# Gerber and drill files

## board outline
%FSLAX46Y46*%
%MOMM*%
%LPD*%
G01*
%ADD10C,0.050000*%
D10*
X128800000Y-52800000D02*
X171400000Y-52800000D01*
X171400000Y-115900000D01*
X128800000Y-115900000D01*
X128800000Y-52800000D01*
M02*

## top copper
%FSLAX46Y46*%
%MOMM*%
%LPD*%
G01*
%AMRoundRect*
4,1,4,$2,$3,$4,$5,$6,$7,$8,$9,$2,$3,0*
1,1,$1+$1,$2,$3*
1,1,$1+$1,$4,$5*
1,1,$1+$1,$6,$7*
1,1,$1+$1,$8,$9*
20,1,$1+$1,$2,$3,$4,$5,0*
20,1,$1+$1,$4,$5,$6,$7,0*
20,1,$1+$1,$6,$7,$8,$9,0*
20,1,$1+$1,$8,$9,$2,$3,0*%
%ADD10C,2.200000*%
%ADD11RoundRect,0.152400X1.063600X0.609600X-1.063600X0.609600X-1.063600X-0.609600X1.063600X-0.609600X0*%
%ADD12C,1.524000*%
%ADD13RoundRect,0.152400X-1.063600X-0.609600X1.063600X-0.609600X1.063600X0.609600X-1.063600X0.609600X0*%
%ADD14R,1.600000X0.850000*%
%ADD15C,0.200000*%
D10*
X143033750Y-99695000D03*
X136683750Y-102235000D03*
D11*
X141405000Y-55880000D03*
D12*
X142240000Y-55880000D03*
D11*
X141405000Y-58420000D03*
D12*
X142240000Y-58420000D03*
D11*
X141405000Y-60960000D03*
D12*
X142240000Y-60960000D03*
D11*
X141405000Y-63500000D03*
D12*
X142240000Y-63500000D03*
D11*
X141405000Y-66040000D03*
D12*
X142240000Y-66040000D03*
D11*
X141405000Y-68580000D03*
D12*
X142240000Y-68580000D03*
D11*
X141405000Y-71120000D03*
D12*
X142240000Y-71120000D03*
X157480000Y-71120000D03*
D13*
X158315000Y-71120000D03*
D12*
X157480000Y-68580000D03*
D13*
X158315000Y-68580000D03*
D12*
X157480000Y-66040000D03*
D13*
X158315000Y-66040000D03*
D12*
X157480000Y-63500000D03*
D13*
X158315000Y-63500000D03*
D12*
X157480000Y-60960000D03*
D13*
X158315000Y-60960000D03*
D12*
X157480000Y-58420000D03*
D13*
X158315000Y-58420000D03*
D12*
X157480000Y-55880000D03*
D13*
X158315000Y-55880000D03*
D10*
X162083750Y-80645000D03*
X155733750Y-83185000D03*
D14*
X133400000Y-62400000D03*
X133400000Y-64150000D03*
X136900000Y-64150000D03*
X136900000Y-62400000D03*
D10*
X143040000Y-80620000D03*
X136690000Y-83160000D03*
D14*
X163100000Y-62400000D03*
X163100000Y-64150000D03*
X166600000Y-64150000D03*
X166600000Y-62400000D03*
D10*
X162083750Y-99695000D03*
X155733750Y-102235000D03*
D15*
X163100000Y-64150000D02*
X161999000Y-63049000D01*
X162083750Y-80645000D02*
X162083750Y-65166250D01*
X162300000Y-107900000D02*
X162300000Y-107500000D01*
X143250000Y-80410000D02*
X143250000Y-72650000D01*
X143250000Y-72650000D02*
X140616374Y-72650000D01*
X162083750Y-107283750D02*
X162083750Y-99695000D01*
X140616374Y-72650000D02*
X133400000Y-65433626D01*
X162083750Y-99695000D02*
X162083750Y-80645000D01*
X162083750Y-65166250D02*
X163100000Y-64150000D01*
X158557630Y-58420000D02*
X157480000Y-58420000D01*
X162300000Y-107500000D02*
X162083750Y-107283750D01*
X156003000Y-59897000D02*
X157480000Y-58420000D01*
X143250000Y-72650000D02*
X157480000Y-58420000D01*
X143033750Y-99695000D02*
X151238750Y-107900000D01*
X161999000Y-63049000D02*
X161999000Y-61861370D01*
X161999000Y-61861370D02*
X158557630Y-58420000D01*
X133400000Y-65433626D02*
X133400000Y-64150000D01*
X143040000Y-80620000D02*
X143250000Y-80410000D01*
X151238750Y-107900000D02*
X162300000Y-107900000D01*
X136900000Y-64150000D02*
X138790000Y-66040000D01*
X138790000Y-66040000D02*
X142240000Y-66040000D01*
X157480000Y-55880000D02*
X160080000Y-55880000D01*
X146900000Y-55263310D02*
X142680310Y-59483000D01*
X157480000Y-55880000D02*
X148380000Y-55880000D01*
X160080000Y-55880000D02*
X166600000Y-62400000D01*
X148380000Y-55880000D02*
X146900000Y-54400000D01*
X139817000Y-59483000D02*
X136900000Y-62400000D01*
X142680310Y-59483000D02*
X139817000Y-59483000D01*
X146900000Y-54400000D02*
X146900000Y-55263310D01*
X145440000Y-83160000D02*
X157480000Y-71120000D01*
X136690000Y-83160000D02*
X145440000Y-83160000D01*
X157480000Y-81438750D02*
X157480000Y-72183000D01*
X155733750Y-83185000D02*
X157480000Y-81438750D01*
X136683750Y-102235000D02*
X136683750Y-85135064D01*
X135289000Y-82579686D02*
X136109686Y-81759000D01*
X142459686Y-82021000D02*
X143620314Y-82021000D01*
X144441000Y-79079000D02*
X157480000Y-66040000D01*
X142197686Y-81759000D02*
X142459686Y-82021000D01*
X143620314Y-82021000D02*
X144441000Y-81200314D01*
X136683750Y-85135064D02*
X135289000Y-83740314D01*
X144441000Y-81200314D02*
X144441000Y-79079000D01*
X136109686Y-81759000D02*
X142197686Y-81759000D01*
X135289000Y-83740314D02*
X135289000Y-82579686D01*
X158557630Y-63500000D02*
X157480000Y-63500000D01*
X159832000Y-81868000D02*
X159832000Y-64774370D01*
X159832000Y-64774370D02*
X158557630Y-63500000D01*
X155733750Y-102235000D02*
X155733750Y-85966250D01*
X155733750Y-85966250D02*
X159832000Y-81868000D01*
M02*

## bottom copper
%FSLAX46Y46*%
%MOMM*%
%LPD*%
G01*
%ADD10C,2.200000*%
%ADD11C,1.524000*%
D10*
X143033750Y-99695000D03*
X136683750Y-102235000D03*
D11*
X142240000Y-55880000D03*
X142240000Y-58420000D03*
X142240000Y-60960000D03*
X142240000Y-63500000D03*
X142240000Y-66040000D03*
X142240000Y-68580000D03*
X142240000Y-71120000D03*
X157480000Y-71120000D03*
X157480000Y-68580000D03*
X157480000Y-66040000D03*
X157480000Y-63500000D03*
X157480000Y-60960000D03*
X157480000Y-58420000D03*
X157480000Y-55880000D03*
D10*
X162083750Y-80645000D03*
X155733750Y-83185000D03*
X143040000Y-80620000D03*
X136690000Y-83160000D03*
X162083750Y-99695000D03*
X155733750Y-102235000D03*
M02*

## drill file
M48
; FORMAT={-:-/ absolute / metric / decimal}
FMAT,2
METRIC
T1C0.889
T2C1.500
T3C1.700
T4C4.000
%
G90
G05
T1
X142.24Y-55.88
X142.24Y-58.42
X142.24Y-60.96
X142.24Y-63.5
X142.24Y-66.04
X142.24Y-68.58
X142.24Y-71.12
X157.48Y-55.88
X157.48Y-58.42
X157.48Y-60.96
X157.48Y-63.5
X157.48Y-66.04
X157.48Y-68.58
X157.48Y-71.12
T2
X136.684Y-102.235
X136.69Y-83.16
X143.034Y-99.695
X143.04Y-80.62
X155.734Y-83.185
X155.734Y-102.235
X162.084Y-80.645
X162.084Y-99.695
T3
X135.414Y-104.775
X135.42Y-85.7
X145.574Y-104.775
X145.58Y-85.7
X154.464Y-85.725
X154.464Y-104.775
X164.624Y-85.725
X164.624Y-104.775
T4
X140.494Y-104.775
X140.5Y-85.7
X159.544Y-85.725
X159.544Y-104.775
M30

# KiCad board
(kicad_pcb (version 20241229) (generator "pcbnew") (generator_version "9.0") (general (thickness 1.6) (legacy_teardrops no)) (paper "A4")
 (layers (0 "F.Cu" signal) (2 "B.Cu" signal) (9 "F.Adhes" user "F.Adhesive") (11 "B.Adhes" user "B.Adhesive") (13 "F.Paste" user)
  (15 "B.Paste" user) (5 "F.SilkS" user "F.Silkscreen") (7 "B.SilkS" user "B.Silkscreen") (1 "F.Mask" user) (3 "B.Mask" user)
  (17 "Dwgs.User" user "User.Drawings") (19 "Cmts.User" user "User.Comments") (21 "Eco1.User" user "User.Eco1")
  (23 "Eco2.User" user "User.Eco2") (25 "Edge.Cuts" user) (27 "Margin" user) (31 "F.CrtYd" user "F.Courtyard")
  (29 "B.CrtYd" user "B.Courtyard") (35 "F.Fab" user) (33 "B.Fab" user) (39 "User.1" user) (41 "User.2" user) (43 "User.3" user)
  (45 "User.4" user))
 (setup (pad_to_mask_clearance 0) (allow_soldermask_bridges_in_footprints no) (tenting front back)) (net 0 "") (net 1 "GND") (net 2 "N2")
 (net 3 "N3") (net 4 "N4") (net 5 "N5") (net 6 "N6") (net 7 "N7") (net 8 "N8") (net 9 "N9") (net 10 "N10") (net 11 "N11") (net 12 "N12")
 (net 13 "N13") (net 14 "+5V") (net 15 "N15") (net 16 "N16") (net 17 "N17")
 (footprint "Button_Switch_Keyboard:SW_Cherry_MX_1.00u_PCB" (layer "F.Cu") (at 143.03375 99.695)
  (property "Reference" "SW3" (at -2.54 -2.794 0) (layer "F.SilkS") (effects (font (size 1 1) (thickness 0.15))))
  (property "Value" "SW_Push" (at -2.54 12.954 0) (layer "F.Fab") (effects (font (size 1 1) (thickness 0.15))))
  (pad "" np_thru_hole circle (at -7.62 5.08) (size 1.7 1.7) (drill 1.7) (layers "*.Cu" "*.Mask"))
  (pad "" np_thru_hole circle (at -2.54 5.08) (size 4 4) (drill 4) (layers "*.Cu" "*.Mask"))
  (pad "" np_thru_hole circle (at 2.54 5.08) (size 1.7 1.7) (drill 1.7) (layers "*.Cu" "*.Mask"))
  (pad "1" thru_hole circle (at 0 0) (size 2.2 2.2) (drill 1.5) (layers "*.Cu" "*.Mask") (remove_unused_layers no) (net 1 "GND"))
  (pad "2" thru_hole circle (at -6.35 2.54) (size 2.2 2.2) (drill 1.5) (layers "*.Cu" "*.Mask") (remove_unused_layers no) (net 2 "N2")))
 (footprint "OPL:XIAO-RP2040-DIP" (layer "F.Cu") (at 149.86 63.5)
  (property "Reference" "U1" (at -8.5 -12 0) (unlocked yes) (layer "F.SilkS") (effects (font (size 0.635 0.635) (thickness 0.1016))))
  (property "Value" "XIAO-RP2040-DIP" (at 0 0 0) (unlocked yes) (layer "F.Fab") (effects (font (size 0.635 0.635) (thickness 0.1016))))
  (pad "1" smd roundrect (at -8.455 -7.62 180) (size 2.432 1.524) (layers "F.Cu" "F.Mask") (roundrect_rratio 0.1) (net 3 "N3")
   (thermal_bridge_angle 45))
  (pad "1" thru_hole circle (at -7.62 -7.62 180) (size 1.524 1.524) (drill 0.889) (layers "*.Cu" "*.Mask") (remove_unused_layers no)
   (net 3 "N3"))
  (pad "2" smd roundrect (at -8.455 -5.08 180) (size 2.432 1.524) (layers "F.Cu" "F.Mask") (roundrect_rratio 0.1) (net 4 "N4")
   (thermal_bridge_angle 45))
  (pad "2" thru_hole circle (at -7.62 -5.08 180) (size 1.524 1.524) (drill 0.889) (layers "*.Cu" "*.Mask") (remove_unused_layers no)
   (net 4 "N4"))
  (pad "3" smd roundrect (at -8.455 -2.54 180) (size 2.432 1.524) (layers "F.Cu" "F.Mask") (roundrect_rratio 0.1) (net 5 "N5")
   (thermal_bridge_angle 45))
  (pad "3" thru_hole circle (at -7.62 -2.54 180) (size 1.524 1.524) (drill 0.889) (layers "*.Cu" "*.Mask") (remove_unused_layers no)
   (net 5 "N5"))
  (pad "4" smd roundrect (at -8.455 0 180) (size 2.432 1.524) (layers "F.Cu" "F.Mask") (roundrect_rratio 0.1) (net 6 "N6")
   (thermal_bridge_angle 45))
  (pad "4" thru_hole circle (at -7.62 0 180) (size 1.524 1.524) (drill 0.889) (layers "*.Cu" "*.Mask") (remove_unused_layers no)
   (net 6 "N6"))
  (pad "5" smd roundrect (at -8.455 2.54 180) (size 2.432 1.524) (layers "F.Cu" "F.Mask") (roundrect_rratio 0.1) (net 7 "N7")
   (thermal_bridge_angle 45))
  (pad "5" thru_hole circle (at -7.62 2.54 180) (size 1.524 1.524) (drill 0.889) (layers "*.Cu" "*.Mask") (remove_unused_layers no)
   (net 7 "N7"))
  (pad "6" smd roundrect (at -8.455 5.08 180) (size 2.432 1.524) (layers "F.Cu" "F.Mask") (roundrect_rratio 0.1) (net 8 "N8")
   (thermal_bridge_angle 45))
  (pad "6" thru_hole circle (at -7.62 5.08 180) (size 1.524 1.524) (drill 0.889) (layers "*.Cu" "*.Mask") (remove_unused_layers no)
   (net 8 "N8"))
  (pad "7" smd roundrect (at -8.455 7.62 180) (size 2.432 1.524) (layers "F.Cu" "F.Mask") (roundrect_rratio 0.1) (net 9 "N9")
   (thermal_bridge_angle 45))
  (pad "7" thru_hole circle (at -7.62 7.62 180) (size 1.524 1.524) (drill 0.889) (layers "*.Cu" "*.Mask") (remove_unused_layers no)
   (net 9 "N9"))
  (pad "8" thru_hole circle (at 7.62 7.62) (size 1.524 1.524) (drill 0.889) (layers "*.Cu" "*.Mask") (remove_unused_layers no)
   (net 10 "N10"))
  (pad "8" smd roundrect (at 8.455 7.62) (size 2.432 1.524) (layers "F.Cu" "F.Mask") (roundrect_rratio 0.1) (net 10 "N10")
   (thermal_bridge_angle 45))
  (pad "9" thru_hole circle (at 7.62 5.08) (size 1.524 1.524) (drill 0.889) (layers "*.Cu" "*.Mask") (remove_unused_layers no)
   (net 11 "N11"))
  (pad "9" smd roundrect (at 8.455 5.08) (size 2.432 1.524) (layers "F.Cu" "F.Mask") (roundrect_rratio 0.1) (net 11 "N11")
   (thermal_bridge_angle 45))
  (pad "10" thru_hole circle (at 7.62 2.54) (size 1.524 1.524) (drill 0.889) (layers "*.Cu" "*.Mask") (remove_unused_layers no) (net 2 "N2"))
  (pad "10" smd roundrect (at 8.455 2.54) (size 2.432 1.524) (layers "F.Cu" "F.Mask") (roundrect_rratio 0.1) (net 2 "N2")
   (thermal_bridge_angle 45))
  (pad "11" thru_hole circle (at 7.62 0) (size 1.524 1.524) (drill 0.889) (layers "*.Cu" "*.Mask") (remove_unused_layers no) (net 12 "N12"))
  (pad "11" smd roundrect (at 8.455 0) (size 2.432 1.524) (layers "F.Cu" "F.Mask") (roundrect_rratio 0.1) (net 12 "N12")
   (thermal_bridge_angle 45))
  (pad "12" thru_hole circle (at 7.62 -2.54) (size 1.524 1.524) (drill 0.889) (layers "*.Cu" "*.Mask") (remove_unused_layers no)
   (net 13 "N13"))
  (pad "12" smd roundrect (at 8.455 -2.54) (size 2.432 1.524) (layers "F.Cu" "F.Mask") (roundrect_rratio 0.1) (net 13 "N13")
   (thermal_bridge_angle 45))
  (pad "13" thru_hole circle (at 7.62 -5.08) (size 1.524 1.524) (drill 0.889) (layers "*.Cu" "*.Mask") (remove_unused_layers no)
   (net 1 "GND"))
  (pad "13" smd roundrect (at 8.455 -5.08) (size 2.432 1.524) (layers "F.Cu" "F.Mask") (roundrect_rratio 0.1) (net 1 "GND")
   (thermal_bridge_angle 45))
  (pad "14" thru_hole circle (at 7.62 -7.62) (size 1.524 1.524) (drill 0.889) (layers "*.Cu" "*.Mask") (remove_unused_layers no)
   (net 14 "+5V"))
  (pad "14" smd roundrect (at 8.455 -7.62) (size 2.432 1.524) (layers "F.Cu" "F.Mask") (roundrect_rratio 0.1) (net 14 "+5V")
   (thermal_bridge_angle 45)))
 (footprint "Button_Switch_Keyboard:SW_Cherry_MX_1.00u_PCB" (layer "F.Cu") (at 162.08375 80.645)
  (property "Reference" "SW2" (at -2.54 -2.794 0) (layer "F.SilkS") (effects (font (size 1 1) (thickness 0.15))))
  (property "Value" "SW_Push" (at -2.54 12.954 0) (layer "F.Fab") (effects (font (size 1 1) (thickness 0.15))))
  (pad "" np_thru_hole circle (at -7.62 5.08) (size 1.7 1.7) (drill 1.7) (layers "*.Cu" "*.Mask"))
  (pad "" np_thru_hole circle (at -2.54 5.08) (size 4 4) (drill 4) (layers "*.Cu" "*.Mask"))
  (pad "" np_thru_hole circle (at 2.54 5.08) (size 1.7 1.7) (drill 1.7) (layers "*.Cu" "*.Mask"))
  (pad "1" thru_hole circle (at 0 0) (size 2.2 2.2) (drill 1.5) (layers "*.Cu" "*.Mask") (remove_unused_layers no) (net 1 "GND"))
  (pad "2" thru_hole circle (at -6.35 2.54) (size 2.2 2.2) (drill 1.5) (layers "*.Cu" "*.Mask") (remove_unused_layers no) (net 11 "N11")))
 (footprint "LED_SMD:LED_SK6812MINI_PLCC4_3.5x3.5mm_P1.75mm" (layer "F.Cu") (at 135.15 63.275)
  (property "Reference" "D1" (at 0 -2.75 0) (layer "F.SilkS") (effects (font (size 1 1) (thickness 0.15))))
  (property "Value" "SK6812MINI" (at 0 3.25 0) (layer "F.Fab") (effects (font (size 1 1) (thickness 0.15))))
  (pad "1" smd rect (at -1.75 -0.875) (size 1.6 0.85) (layers "F.Cu" "F.Mask" "F.Paste") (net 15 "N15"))
  (pad "2" smd rect (at -1.75 0.875) (size 1.6 0.85) (layers "F.Cu" "F.Mask" "F.Paste") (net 1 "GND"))
  (pad "3" smd rect (at 1.75 0.875) (size 1.6 0.85) (layers "F.Cu" "F.Mask" "F.Paste") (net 7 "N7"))
  (pad "4" smd rect (at 1.75 -0.875) (size 1.6 0.85) (layers "F.Cu" "F.Mask" "F.Paste") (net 14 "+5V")))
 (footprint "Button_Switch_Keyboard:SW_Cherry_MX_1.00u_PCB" (layer "F.Cu") (at 143.04 80.62)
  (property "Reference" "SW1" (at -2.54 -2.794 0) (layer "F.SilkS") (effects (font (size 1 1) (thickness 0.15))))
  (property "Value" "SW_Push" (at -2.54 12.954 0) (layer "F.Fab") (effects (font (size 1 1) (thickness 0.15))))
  (pad "" np_thru_hole circle (at -7.62 5.08) (size 1.7 1.7) (drill 1.7) (layers "*.Cu" "*.Mask"))
  (pad "" np_thru_hole circle (at -2.54 5.08) (size 4 4) (drill 4) (layers "*.Cu" "*.Mask"))
  (pad "" np_thru_hole circle (at 2.54 5.08) (size 1.7 1.7) (drill 1.7) (layers "*.Cu" "*.Mask"))
  (pad "1" thru_hole circle (at 0 0) (size 2.2 2.2) (drill 1.5) (layers "*.Cu" "*.Mask") (remove_unused_layers no) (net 1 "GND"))
  (pad "2" thru_hole circle (at -6.35 2.54) (size 2.2 2.2) (drill 1.5) (layers "*.Cu" "*.Mask") (remove_unused_layers no) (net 10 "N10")))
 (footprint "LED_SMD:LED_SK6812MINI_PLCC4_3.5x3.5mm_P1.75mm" (layer "F.Cu") (at 164.85 63.275)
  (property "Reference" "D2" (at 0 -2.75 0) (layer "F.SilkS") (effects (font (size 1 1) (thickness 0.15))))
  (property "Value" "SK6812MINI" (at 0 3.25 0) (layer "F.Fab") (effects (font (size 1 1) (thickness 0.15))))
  (pad "1" smd rect (at -1.75 -0.875) (size 1.6 0.85) (layers "F.Cu" "F.Mask" "F.Paste") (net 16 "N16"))
  (pad "2" smd rect (at -1.75 0.875) (size 1.6 0.85) (layers "F.Cu" "F.Mask" "F.Paste") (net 1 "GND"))
  (pad "3" smd rect (at 1.75 0.875) (size 1.6 0.85) (layers "F.Cu" "F.Mask" "F.Paste") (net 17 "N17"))
  (pad "4" smd rect (at 1.75 -0.875) (size 1.6 0.85) (layers "F.Cu" "F.Mask" "F.Paste") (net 14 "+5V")))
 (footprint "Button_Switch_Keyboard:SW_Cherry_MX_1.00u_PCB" (layer "F.Cu") (at 162.08375 99.695)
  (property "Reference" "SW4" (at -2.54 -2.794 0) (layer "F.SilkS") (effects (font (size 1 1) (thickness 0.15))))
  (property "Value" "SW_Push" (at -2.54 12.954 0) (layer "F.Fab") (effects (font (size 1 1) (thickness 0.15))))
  (pad "" np_thru_hole circle (at -7.62 5.08) (size 1.7 1.7) (drill 1.7) (layers "*.Cu" "*.Mask"))
  (pad "" np_thru_hole circle (at -2.54 5.08) (size 4 4) (drill 4) (layers "*.Cu" "*.Mask"))
  (pad "" np_thru_hole circle (at 2.54 5.08) (size 1.7 1.7) (drill 1.7) (layers "*.Cu" "*.Mask"))
  (pad "1" thru_hole circle (at 0 0) (size 2.2 2.2) (drill 1.5) (layers "*.Cu" "*.Mask") (remove_unused_layers no) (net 1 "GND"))
  (pad "2" thru_hole circle (at -6.35 2.54) (size 2.2 2.2) (drill 1.5) (layers "*.Cu" "*.Mask") (remove_unused_layers no) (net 12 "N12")))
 (gr_rect (start 128.8 52.8) (end 171.4 115.9) (stroke (width 0.05) (type default)) (fill no) (layer "Edge.Cuts"))
 (segment (start 163.1 64.15) (end 161.999 63.049) (width 0.2) (layer "F.Cu") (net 1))
 (segment (start 162.08375 80.645) (end 162.08375 65.16625) (width 0.2) (layer "F.Cu") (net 1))
 (segment (start 162.3 107.9) (end 162.3 107.5) (width 0.2) (layer "F.Cu") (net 1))
 (segment (start 143.25 80.41) (end 143.25 72.65) (width 0.2) (layer "F.Cu") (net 1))
 (segment (start 143.25 72.65) (end 140.616374 72.65) (width 0.2) (layer "F.Cu") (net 1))
 (segment (start 162.08375 107.28375) (end 162.08375 99.695) (width 0.2) (layer "F.Cu") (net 1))
 (segment (start 140.616374 72.65) (end 133.4 65.433626) (width 0.2) (layer "F.Cu") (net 1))
 (segment (start 162.08375 99.695) (end 162.08375 80.645) (width 0.2) (layer "F.Cu") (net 1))
 (segment (start 162.08375 65.16625) (end 163.1 64.15) (width 0.2) (layer "F.Cu") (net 1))
 (segment (start 158.55763 58.42) (end 157.48 58.42) (width 0.2) (layer "F.Cu") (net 1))
 (segment (start 162.3 107.5) (end 162.08375 107.28375) (width 0.2) (layer "F.Cu") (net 1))
 (segment (start 156.003 59.897) (end 157.48 58.42) (width 0.2) (layer "F.Cu") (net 1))
 (segment (start 143.25 72.65) (end 157.48 58.42) (width 0.2) (layer "F.Cu") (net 1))
 (segment (start 143.03375 99.695) (end 151.23875 107.9) (width 0.2) (layer "F.Cu") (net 1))
 (segment (start 161.999 63.049) (end 161.999 61.86137) (width 0.2) (layer "F.Cu") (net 1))
 (segment (start 161.999 61.86137) (end 158.55763 58.42) (width 0.2) (layer "F.Cu") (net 1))
 (segment (start 133.4 65.433626) (end 133.4 64.15) (width 0.2) (layer "F.Cu") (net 1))
 (segment (start 143.04 80.62) (end 143.25 80.41) (width 0.2) (layer "F.Cu") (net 1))
 (segment (start 151.23875 107.9) (end 162.3 107.9) (width 0.2) (layer "F.Cu") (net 1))
 (segment (start 136.9 64.15) (end 138.79 66.04) (width 0.2) (layer "F.Cu") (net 7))
 (segment (start 138.79 66.04) (end 142.24 66.04) (width 0.2) (layer "F.Cu") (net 7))
 (segment (start 157.48 55.88) (end 160.08 55.88) (width 0.2) (layer "F.Cu") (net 14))
 (segment (start 146.9 55.26331) (end 142.68031 59.483) (width 0.2) (layer "F.Cu") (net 14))
 (segment (start 157.48 55.88) (end 148.38 55.88) (width 0.2) (layer "F.Cu") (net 14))
 (segment (start 160.08 55.88) (end 166.6 62.4) (width 0.2) (layer "F.Cu") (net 14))
 (segment (start 148.38 55.88) (end 146.9 54.4) (width 0.2) (layer "F.Cu") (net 14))
 (segment (start 139.817 59.483) (end 136.9 62.4) (width 0.2) (layer "F.Cu") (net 14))
 (segment (start 142.68031 59.483) (end 139.817 59.483) (width 0.2) (layer "F.Cu") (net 14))
 (segment (start 146.9 54.4) (end 146.9 55.26331) (width 0.2) (layer "F.Cu") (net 14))
 (segment (start 145.44 83.16) (end 157.48 71.12) (width 0.2) (layer "F.Cu") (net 10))
 (segment (start 136.69 83.16) (end 145.44 83.16) (width 0.2) (layer "F.Cu") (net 10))
 (segment (start 157.48 81.43875) (end 157.48 72.183) (width 0.2) (layer "F.Cu") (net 11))
 (segment (start 155.73375 83.185) (end 157.48 81.43875) (width 0.2) (layer "F.Cu") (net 11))
 (segment (start 136.68375 102.235) (end 136.68375 85.135064) (width 0.2) (layer "F.Cu") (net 2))
 (segment (start 135.289 82.579686) (end 136.109686 81.759) (width 0.2) (layer "F.Cu") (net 2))
 (segment (start 142.459686 82.021) (end 143.620314 82.021) (width 0.2) (layer "F.Cu") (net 2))
 (segment (start 144.441 79.079) (end 157.48 66.04) (width 0.2) (layer "F.Cu") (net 2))
 (segment (start 142.197686 81.759) (end 142.459686 82.021) (width 0.2) (layer "F.Cu") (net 2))
 (segment (start 143.620314 82.021) (end 144.441 81.200314) (width 0.2) (layer "F.Cu") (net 2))
 (segment (start 136.68375 85.135064) (end 135.289 83.740314) (width 0.2) (layer "F.Cu") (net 2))
 (segment (start 144.441 81.200314) (end 144.441 79.079) (width 0.2) (layer "F.Cu") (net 2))
 (segment (start 136.109686 81.759) (end 142.197686 81.759) (width 0.2) (layer "F.Cu") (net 2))
 (segment (start 135.289 83.740314) (end 135.289 82.579686) (width 0.2) (layer "F.Cu") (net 2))
 (segment (start 158.55763 63.5) (end 157.48 63.5) (width 0.2) (layer "F.Cu") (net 12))
 (segment (start 159.832 81.868) (end 159.832 64.77437) (width 0.2) (layer "F.Cu") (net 12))
 (segment (start 159.832 64.77437) (end 158.55763 63.5) (width 0.2) (layer "F.Cu") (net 12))
 (segment (start 155.73375 102.235) (end 155.73375 85.96625) (width 0.2) (layer "F.Cu") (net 12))
 (segment (start 155.73375 85.96625) (end 159.832 81.868) (width 0.2) (layer "F.Cu") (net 12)))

